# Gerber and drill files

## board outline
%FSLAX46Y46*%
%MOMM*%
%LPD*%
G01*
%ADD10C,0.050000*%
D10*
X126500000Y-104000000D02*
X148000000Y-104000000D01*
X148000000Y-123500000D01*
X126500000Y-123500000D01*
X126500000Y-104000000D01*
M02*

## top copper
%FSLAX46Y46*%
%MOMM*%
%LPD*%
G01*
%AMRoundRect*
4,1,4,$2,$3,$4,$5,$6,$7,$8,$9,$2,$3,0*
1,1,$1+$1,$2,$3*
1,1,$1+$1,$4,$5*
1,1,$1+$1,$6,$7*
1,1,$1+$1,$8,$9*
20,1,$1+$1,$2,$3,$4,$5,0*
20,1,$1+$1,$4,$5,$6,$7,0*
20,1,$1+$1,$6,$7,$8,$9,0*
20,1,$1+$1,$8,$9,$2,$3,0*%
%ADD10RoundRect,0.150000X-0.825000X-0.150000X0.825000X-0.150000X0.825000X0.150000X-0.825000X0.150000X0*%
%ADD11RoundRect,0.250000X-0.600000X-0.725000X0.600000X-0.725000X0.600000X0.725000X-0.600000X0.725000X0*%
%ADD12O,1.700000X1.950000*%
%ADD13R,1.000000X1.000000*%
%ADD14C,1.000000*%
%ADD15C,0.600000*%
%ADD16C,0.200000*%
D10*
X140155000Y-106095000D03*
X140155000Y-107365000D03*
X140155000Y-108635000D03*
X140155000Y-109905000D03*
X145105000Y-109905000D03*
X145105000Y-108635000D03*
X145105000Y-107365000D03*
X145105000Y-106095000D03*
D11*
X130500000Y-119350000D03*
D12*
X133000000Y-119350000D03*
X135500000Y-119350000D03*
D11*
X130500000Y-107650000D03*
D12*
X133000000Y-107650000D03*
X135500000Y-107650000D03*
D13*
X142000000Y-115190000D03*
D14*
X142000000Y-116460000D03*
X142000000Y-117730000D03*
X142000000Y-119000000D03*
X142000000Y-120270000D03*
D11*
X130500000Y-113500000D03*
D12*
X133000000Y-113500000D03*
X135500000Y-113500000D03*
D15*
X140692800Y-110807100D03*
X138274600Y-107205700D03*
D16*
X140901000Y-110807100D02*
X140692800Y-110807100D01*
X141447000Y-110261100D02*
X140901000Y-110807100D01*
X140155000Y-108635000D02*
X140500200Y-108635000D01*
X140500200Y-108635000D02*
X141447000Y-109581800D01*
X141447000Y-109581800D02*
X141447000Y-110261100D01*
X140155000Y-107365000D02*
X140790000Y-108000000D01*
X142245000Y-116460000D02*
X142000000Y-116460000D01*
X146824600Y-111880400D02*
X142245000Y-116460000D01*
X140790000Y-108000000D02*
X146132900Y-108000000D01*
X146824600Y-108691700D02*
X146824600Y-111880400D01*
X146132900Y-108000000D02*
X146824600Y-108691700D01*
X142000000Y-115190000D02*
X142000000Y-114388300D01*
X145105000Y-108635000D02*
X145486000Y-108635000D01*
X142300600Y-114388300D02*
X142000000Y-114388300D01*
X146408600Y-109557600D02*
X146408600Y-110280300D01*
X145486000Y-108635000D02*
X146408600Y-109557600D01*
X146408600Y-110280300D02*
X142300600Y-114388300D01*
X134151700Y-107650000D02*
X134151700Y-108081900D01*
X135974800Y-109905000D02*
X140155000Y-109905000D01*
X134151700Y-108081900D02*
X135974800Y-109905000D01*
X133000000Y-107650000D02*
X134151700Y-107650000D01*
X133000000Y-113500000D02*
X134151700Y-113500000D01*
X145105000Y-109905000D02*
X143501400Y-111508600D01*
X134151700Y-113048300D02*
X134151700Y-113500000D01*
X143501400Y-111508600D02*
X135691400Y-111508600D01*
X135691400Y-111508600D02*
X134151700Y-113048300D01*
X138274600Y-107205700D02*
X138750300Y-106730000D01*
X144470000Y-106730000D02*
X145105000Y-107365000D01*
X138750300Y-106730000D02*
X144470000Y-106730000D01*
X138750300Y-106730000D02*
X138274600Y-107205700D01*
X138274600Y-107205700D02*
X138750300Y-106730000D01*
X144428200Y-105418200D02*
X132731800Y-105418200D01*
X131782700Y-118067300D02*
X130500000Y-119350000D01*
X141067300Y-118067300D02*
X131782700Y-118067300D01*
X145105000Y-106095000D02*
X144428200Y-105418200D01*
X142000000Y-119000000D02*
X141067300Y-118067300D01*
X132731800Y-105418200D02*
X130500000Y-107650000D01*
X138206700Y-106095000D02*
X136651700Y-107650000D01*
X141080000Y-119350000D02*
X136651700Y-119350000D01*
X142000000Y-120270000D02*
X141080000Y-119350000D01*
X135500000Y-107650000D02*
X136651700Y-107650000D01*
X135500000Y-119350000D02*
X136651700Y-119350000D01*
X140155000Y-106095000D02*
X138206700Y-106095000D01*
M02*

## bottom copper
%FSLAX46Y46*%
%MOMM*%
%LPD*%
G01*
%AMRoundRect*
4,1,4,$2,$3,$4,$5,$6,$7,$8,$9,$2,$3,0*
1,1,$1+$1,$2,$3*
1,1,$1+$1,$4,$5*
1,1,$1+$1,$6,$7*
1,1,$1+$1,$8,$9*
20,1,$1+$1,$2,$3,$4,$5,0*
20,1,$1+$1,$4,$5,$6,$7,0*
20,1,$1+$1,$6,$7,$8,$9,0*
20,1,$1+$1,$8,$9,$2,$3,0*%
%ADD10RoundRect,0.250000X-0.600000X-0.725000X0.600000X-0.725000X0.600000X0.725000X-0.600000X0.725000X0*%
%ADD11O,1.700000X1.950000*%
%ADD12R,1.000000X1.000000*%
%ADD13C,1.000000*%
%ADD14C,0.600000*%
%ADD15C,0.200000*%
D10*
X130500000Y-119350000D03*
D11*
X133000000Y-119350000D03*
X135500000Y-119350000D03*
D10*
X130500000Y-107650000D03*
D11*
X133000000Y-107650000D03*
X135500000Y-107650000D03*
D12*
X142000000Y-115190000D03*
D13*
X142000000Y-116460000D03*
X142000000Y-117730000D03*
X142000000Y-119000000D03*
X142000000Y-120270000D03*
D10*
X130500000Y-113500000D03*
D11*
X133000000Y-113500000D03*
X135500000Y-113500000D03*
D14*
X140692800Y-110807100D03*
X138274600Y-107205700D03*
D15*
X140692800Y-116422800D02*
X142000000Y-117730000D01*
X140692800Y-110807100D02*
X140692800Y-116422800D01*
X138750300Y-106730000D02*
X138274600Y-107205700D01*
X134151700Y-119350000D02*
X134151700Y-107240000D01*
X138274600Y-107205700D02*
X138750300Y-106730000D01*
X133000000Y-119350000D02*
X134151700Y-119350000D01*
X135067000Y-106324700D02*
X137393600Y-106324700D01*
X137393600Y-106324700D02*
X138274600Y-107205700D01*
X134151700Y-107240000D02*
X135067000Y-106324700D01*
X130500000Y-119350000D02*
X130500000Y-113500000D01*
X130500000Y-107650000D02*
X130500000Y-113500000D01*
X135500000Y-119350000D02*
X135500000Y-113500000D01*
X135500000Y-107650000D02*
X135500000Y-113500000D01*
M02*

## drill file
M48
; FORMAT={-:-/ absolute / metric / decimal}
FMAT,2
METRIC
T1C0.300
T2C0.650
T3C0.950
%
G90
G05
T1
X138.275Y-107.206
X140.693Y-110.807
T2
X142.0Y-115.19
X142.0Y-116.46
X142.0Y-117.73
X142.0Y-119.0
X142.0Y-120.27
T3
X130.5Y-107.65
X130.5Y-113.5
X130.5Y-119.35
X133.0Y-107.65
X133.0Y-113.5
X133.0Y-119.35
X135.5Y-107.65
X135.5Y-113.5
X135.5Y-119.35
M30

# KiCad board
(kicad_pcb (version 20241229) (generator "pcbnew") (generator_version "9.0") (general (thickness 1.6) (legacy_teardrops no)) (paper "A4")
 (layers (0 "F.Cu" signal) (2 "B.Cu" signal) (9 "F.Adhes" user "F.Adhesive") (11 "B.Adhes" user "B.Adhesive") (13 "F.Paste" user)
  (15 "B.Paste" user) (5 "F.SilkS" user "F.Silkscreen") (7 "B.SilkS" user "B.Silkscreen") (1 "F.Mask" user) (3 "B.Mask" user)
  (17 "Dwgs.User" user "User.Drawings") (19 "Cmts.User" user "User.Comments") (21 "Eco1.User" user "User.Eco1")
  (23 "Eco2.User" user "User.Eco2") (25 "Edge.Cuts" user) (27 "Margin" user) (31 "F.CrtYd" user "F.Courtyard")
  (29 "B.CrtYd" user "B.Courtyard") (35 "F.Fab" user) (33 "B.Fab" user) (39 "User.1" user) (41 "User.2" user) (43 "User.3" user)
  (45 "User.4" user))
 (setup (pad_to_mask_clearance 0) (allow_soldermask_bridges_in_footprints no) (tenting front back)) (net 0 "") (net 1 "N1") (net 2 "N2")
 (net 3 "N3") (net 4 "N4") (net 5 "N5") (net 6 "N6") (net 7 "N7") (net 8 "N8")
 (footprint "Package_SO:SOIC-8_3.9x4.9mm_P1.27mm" (layer "F.Cu") (at 142.63 108)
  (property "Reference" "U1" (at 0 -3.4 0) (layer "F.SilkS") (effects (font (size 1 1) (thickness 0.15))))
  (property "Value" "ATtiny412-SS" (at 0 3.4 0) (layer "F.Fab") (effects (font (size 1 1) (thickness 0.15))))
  (pad "1" smd roundrect (at -2.475 -1.905) (size 1.95 0.6) (layers "F.Cu" "F.Mask" "F.Paste") (roundrect_rratio 0.25) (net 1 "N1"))
  (pad "2" smd roundrect (at -2.475 -0.635) (size 1.95 0.6) (layers "F.Cu" "F.Mask" "F.Paste") (roundrect_rratio 0.25) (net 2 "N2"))
  (pad "3" smd roundrect (at -2.475 0.635) (size 1.95 0.6) (layers "F.Cu" "F.Mask" "F.Paste") (roundrect_rratio 0.25) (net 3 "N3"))
  (pad "4" smd roundrect (at -2.475 1.905) (size 1.95 0.6) (layers "F.Cu" "F.Mask" "F.Paste") (roundrect_rratio 0.25) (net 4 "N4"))
  (pad "5" smd roundrect (at 2.475 1.905) (size 1.95 0.6) (layers "F.Cu" "F.Mask" "F.Paste") (roundrect_rratio 0.25) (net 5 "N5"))
  (pad "6" smd roundrect (at 2.475 0.635) (size 1.95 0.6) (layers "F.Cu" "F.Mask" "F.Paste") (roundrect_rratio 0.25) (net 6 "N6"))
  (pad "7" smd roundrect (at 2.475 -0.635) (size 1.95 0.6) (layers "F.Cu" "F.Mask" "F.Paste") (roundrect_rratio 0.25) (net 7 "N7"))
  (pad "8" smd roundrect (at 2.475 -1.905) (size 1.95 0.6) (layers "F.Cu" "F.Mask" "F.Paste") (roundrect_rratio 0.25) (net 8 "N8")))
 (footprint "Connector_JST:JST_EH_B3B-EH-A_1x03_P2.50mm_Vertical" (layer "F.Cu") (at 130.5 119.35)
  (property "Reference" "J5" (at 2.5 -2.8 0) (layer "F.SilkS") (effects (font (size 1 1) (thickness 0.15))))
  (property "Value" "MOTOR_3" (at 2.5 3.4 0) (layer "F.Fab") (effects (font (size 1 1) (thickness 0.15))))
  (pad "1" thru_hole roundrect (at 0 0) (size 1.7 1.95) (drill 0.95) (layers "*.Cu" "*.Mask") (remove_unused_layers no)
   (roundrect_rratio 0.147059) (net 8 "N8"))
  (pad "2" thru_hole oval (at 2.5 0) (size 1.7 1.95) (drill 0.95) (layers "*.Cu" "*.Mask") (remove_unused_layers no) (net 7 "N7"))
  (pad "3" thru_hole oval (at 5 0) (size 1.7 1.95) (drill 0.95) (layers "*.Cu" "*.Mask") (remove_unused_layers no) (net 1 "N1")))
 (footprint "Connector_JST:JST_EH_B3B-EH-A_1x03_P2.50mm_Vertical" (layer "F.Cu") (at 130.5 107.65)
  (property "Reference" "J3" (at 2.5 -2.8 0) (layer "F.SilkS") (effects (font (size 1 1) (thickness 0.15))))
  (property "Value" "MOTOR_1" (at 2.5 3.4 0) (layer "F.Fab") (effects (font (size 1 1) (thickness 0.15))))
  (pad "1" thru_hole roundrect (at 0 0) (size 1.7 1.95) (drill 0.95) (layers "*.Cu" "*.Mask") (remove_unused_layers no)
   (roundrect_rratio 0.147059) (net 8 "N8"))
  (pad "2" thru_hole oval (at 2.5 0) (size 1.7 1.95) (drill 0.95) (layers "*.Cu" "*.Mask") (remove_unused_layers no) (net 4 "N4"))
  (pad "3" thru_hole oval (at 5 0) (size 1.7 1.95) (drill 0.95) (layers "*.Cu" "*.Mask") (remove_unused_layers no) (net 1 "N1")))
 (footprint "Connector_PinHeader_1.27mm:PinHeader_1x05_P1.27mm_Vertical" (layer "F.Cu") (at 142 115.19)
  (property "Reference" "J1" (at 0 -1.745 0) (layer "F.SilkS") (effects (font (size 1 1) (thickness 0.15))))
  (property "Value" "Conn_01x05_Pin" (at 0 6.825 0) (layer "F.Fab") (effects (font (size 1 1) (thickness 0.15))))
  (pad "1" thru_hole rect (at 0 0) (size 1 1) (drill 0.65) (layers "*.Cu" "*.Mask") (remove_unused_layers no) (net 6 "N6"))
  (pad "2" thru_hole circle (at 0 1.27) (size 1 1) (drill 0.65) (layers "*.Cu" "*.Mask") (remove_unused_layers no) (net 2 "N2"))
  (pad "3" thru_hole circle (at 0 2.54) (size 1 1) (drill 0.65) (layers "*.Cu" "*.Mask") (remove_unused_layers no) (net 3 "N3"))
  (pad "4" thru_hole circle (at 0 3.81) (size 1 1) (drill 0.65) (layers "*.Cu" "*.Mask") (remove_unused_layers no) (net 8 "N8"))
  (pad "5" thru_hole circle (at 0 5.08) (size 1 1) (drill 0.65) (layers "*.Cu" "*.Mask") (remove_unused_layers no) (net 1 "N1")))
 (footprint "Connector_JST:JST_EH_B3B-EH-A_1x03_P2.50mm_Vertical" (layer "F.Cu") (at 130.5 113.5)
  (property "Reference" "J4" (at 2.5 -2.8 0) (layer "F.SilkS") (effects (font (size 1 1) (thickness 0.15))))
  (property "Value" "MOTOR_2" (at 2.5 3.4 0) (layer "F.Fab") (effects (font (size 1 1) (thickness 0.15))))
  (pad "1" thru_hole roundrect (at 0 0) (size 1.7 1.95) (drill 0.95) (layers "*.Cu" "*.Mask") (remove_unused_layers no)
   (roundrect_rratio 0.147059) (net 8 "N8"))
  (pad "2" thru_hole oval (at 2.5 0) (size 1.7 1.95) (drill 0.95) (layers "*.Cu" "*.Mask") (remove_unused_layers no) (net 5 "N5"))
  (pad "3" thru_hole oval (at 5 0) (size 1.7 1.95) (drill 0.95) (layers "*.Cu" "*.Mask") (remove_unused_layers no) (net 1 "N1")))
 (gr_rect (start 126.5 104) (end 148 123.5) (stroke (width 0.05) (type default)) (fill no) (layer "Edge.Cuts"))
 (segment (start 140.901 110.8071) (end 140.6928 110.8071) (width 0.2) (layer "F.Cu") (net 3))
 (segment (start 141.447 110.2611) (end 140.901 110.8071) (width 0.2) (layer "F.Cu") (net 3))
 (segment (start 140.155 108.635) (end 140.5002 108.635) (width 0.2) (layer "F.Cu") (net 3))
 (segment (start 140.5002 108.635) (end 141.447 109.5818) (width 0.2) (layer "F.Cu") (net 3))
 (segment (start 141.447 109.5818) (end 141.447 110.2611) (width 0.2) (layer "F.Cu") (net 3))
 (via (at 140.6928 110.8071) (size 0.6) (drill 0.3) (layers "F.Cu" "B.Cu") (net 3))
 (segment (start 140.6928 116.4228) (end 142 117.73) (width 0.2) (layer "B.Cu") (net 3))
 (segment (start 140.6928 110.8071) (end 140.6928 116.4228) (width 0.2) (layer "B.Cu") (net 3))
 (segment (start 140.155 107.365) (end 140.79 108) (width 0.2) (layer "F.Cu") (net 2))
 (segment (start 142.245 116.46) (end 142 116.46) (width 0.2) (layer "F.Cu") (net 2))
 (segment (start 146.8246 111.8804) (end 142.245 116.46) (width 0.2) (layer "F.Cu") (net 2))
 (segment (start 140.79 108) (end 146.1329 108) (width 0.2) (layer "F.Cu") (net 2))
 (segment (start 146.8246 108.6917) (end 146.8246 111.8804) (width 0.2) (layer "F.Cu") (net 2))
 (segment (start 146.1329 108) (end 146.8246 108.6917) (width 0.2) (layer "F.Cu") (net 2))
 (segment (start 142 115.19) (end 142 114.3883) (width 0.2) (layer "F.Cu") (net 6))
 (segment (start 145.105 108.635) (end 145.486 108.635) (width 0.2) (layer "F.Cu") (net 6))
 (segment (start 142.3006 114.3883) (end 142 114.3883) (width 0.2) (layer "F.Cu") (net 6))
 (segment (start 146.4086 109.5576) (end 146.4086 110.2803) (width 0.2) (layer "F.Cu") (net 6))
 (segment (start 145.486 108.635) (end 146.4086 109.5576) (width 0.2) (layer "F.Cu") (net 6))
 (segment (start 146.4086 110.2803) (end 142.3006 114.3883) (width 0.2) (layer "F.Cu") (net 6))
 (segment (start 134.1517 107.65) (end 134.1517 108.0819) (width 0.2) (layer "F.Cu") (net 4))
 (segment (start 135.9748 109.905) (end 140.155 109.905) (width 0.2) (layer "F.Cu") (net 4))
 (segment (start 134.1517 108.0819) (end 135.9748 109.905) (width 0.2) (layer "F.Cu") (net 4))
 (segment (start 133 107.65) (end 134.1517 107.65) (width 0.2) (layer "F.Cu") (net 4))
 (segment (start 133 113.5) (end 134.1517 113.5) (width 0.2) (layer "F.Cu") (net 5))
 (segment (start 145.105 109.905) (end 143.5014 111.5086) (width 0.2) (layer "F.Cu") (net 5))
 (segment (start 134.1517 113.0483) (end 134.1517 113.5) (width 0.2) (layer "F.Cu") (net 5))
 (segment (start 143.5014 111.5086) (end 135.6914 111.5086) (width 0.2) (layer "F.Cu") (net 5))
 (segment (start 135.6914 111.5086) (end 134.1517 113.0483) (width 0.2) (layer "F.Cu") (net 5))
 (segment (start 138.2746 107.2057) (end 138.7503 106.73) (width 0.2) (layer "F.Cu") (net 7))
 (segment (start 144.47 106.73) (end 145.105 107.365) (width 0.2) (layer "F.Cu") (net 7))
 (segment (start 138.7503 106.73) (end 144.47 106.73) (width 0.2) (layer "F.Cu") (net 7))
 (segment (start 138.7503 106.73) (end 138.2746 107.2057) (width 0.2) (layer "F.Cu") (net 7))
 (segment (start 138.2746 107.2057) (end 138.7503 106.73) (width 0.2) (layer "F.Cu") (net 7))
 (via (at 138.2746 107.2057) (size 0.6) (drill 0.3) (layers "F.Cu" "B.Cu") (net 7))
 (segment (start 138.7503 106.73) (end 138.2746 107.2057) (width 0.2) (layer "B.Cu") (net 7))
 (segment (start 134.1517 119.35) (end 134.1517 107.24) (width 0.2) (layer "B.Cu") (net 7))
 (segment (start 138.2746 107.2057) (end 138.7503 106.73) (width 0.2) (layer "B.Cu") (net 7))
 (segment (start 133 119.35) (end 134.1517 119.35) (width 0.2) (layer "B.Cu") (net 7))
 (segment (start 135.067 106.3247) (end 137.3936 106.3247) (width 0.2) (layer "B.Cu") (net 7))
 (segment (start 137.3936 106.3247) (end 138.2746 107.2057) (width 0.2) (layer "B.Cu") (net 7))
 (segment (start 134.1517 107.24) (end 135.067 106.3247) (width 0.2) (layer "B.Cu") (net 7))
 (segment (start 144.4282 105.4182) (end 132.7318 105.4182) (width 0.2) (layer "F.Cu") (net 8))
 (segment (start 131.7827 118.0673) (end 130.5 119.35) (width 0.2) (layer "F.Cu") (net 8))
 (segment (start 141.0673 118.0673) (end 131.7827 118.0673) (width 0.2) (layer "F.Cu") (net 8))
 (segment (start 145.105 106.095) (end 144.4282 105.4182) (width 0.2) (layer "F.Cu") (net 8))
 (segment (start 142 119) (end 141.0673 118.0673) (width 0.2) (layer "F.Cu") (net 8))
 (segment (start 132.7318 105.4182) (end 130.5 107.65) (width 0.2) (layer "F.Cu") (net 8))
 (segment (start 130.5 119.35) (end 130.5 113.5) (width 0.2) (layer "B.Cu") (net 8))
 (segment (start 130.5 107.65) (end 130.5 113.5) (width 0.2) (layer "B.Cu") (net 8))
 (segment (start 138.2067 106.095) (end 136.6517 107.65) (width 0.2) (layer "F.Cu") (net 1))
 (segment (start 141.08 119.35) (end 136.6517 119.35) (width 0.2) (layer "F.Cu") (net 1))
 (segment (start 142 120.27) (end 141.08 119.35) (width 0.2) (layer "F.Cu") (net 1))
 (segment (start 135.5 107.65) (end 136.6517 107.65) (width 0.2) (layer "F.Cu") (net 1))
 (segment (start 135.5 119.35) (end 136.6517 119.35) (width 0.2) (layer "F.Cu") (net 1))
 (segment (start 140.155 106.095) (end 138.2067 106.095) (width 0.2) (layer "F.Cu") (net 1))
 (segment (start 135.5 119.35) (end 135.5 113.5) (width 0.2) (layer "B.Cu") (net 1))
 (segment (start 135.5 107.65) (end 135.5 113.5) (width 0.2) (layer "B.Cu") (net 1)))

